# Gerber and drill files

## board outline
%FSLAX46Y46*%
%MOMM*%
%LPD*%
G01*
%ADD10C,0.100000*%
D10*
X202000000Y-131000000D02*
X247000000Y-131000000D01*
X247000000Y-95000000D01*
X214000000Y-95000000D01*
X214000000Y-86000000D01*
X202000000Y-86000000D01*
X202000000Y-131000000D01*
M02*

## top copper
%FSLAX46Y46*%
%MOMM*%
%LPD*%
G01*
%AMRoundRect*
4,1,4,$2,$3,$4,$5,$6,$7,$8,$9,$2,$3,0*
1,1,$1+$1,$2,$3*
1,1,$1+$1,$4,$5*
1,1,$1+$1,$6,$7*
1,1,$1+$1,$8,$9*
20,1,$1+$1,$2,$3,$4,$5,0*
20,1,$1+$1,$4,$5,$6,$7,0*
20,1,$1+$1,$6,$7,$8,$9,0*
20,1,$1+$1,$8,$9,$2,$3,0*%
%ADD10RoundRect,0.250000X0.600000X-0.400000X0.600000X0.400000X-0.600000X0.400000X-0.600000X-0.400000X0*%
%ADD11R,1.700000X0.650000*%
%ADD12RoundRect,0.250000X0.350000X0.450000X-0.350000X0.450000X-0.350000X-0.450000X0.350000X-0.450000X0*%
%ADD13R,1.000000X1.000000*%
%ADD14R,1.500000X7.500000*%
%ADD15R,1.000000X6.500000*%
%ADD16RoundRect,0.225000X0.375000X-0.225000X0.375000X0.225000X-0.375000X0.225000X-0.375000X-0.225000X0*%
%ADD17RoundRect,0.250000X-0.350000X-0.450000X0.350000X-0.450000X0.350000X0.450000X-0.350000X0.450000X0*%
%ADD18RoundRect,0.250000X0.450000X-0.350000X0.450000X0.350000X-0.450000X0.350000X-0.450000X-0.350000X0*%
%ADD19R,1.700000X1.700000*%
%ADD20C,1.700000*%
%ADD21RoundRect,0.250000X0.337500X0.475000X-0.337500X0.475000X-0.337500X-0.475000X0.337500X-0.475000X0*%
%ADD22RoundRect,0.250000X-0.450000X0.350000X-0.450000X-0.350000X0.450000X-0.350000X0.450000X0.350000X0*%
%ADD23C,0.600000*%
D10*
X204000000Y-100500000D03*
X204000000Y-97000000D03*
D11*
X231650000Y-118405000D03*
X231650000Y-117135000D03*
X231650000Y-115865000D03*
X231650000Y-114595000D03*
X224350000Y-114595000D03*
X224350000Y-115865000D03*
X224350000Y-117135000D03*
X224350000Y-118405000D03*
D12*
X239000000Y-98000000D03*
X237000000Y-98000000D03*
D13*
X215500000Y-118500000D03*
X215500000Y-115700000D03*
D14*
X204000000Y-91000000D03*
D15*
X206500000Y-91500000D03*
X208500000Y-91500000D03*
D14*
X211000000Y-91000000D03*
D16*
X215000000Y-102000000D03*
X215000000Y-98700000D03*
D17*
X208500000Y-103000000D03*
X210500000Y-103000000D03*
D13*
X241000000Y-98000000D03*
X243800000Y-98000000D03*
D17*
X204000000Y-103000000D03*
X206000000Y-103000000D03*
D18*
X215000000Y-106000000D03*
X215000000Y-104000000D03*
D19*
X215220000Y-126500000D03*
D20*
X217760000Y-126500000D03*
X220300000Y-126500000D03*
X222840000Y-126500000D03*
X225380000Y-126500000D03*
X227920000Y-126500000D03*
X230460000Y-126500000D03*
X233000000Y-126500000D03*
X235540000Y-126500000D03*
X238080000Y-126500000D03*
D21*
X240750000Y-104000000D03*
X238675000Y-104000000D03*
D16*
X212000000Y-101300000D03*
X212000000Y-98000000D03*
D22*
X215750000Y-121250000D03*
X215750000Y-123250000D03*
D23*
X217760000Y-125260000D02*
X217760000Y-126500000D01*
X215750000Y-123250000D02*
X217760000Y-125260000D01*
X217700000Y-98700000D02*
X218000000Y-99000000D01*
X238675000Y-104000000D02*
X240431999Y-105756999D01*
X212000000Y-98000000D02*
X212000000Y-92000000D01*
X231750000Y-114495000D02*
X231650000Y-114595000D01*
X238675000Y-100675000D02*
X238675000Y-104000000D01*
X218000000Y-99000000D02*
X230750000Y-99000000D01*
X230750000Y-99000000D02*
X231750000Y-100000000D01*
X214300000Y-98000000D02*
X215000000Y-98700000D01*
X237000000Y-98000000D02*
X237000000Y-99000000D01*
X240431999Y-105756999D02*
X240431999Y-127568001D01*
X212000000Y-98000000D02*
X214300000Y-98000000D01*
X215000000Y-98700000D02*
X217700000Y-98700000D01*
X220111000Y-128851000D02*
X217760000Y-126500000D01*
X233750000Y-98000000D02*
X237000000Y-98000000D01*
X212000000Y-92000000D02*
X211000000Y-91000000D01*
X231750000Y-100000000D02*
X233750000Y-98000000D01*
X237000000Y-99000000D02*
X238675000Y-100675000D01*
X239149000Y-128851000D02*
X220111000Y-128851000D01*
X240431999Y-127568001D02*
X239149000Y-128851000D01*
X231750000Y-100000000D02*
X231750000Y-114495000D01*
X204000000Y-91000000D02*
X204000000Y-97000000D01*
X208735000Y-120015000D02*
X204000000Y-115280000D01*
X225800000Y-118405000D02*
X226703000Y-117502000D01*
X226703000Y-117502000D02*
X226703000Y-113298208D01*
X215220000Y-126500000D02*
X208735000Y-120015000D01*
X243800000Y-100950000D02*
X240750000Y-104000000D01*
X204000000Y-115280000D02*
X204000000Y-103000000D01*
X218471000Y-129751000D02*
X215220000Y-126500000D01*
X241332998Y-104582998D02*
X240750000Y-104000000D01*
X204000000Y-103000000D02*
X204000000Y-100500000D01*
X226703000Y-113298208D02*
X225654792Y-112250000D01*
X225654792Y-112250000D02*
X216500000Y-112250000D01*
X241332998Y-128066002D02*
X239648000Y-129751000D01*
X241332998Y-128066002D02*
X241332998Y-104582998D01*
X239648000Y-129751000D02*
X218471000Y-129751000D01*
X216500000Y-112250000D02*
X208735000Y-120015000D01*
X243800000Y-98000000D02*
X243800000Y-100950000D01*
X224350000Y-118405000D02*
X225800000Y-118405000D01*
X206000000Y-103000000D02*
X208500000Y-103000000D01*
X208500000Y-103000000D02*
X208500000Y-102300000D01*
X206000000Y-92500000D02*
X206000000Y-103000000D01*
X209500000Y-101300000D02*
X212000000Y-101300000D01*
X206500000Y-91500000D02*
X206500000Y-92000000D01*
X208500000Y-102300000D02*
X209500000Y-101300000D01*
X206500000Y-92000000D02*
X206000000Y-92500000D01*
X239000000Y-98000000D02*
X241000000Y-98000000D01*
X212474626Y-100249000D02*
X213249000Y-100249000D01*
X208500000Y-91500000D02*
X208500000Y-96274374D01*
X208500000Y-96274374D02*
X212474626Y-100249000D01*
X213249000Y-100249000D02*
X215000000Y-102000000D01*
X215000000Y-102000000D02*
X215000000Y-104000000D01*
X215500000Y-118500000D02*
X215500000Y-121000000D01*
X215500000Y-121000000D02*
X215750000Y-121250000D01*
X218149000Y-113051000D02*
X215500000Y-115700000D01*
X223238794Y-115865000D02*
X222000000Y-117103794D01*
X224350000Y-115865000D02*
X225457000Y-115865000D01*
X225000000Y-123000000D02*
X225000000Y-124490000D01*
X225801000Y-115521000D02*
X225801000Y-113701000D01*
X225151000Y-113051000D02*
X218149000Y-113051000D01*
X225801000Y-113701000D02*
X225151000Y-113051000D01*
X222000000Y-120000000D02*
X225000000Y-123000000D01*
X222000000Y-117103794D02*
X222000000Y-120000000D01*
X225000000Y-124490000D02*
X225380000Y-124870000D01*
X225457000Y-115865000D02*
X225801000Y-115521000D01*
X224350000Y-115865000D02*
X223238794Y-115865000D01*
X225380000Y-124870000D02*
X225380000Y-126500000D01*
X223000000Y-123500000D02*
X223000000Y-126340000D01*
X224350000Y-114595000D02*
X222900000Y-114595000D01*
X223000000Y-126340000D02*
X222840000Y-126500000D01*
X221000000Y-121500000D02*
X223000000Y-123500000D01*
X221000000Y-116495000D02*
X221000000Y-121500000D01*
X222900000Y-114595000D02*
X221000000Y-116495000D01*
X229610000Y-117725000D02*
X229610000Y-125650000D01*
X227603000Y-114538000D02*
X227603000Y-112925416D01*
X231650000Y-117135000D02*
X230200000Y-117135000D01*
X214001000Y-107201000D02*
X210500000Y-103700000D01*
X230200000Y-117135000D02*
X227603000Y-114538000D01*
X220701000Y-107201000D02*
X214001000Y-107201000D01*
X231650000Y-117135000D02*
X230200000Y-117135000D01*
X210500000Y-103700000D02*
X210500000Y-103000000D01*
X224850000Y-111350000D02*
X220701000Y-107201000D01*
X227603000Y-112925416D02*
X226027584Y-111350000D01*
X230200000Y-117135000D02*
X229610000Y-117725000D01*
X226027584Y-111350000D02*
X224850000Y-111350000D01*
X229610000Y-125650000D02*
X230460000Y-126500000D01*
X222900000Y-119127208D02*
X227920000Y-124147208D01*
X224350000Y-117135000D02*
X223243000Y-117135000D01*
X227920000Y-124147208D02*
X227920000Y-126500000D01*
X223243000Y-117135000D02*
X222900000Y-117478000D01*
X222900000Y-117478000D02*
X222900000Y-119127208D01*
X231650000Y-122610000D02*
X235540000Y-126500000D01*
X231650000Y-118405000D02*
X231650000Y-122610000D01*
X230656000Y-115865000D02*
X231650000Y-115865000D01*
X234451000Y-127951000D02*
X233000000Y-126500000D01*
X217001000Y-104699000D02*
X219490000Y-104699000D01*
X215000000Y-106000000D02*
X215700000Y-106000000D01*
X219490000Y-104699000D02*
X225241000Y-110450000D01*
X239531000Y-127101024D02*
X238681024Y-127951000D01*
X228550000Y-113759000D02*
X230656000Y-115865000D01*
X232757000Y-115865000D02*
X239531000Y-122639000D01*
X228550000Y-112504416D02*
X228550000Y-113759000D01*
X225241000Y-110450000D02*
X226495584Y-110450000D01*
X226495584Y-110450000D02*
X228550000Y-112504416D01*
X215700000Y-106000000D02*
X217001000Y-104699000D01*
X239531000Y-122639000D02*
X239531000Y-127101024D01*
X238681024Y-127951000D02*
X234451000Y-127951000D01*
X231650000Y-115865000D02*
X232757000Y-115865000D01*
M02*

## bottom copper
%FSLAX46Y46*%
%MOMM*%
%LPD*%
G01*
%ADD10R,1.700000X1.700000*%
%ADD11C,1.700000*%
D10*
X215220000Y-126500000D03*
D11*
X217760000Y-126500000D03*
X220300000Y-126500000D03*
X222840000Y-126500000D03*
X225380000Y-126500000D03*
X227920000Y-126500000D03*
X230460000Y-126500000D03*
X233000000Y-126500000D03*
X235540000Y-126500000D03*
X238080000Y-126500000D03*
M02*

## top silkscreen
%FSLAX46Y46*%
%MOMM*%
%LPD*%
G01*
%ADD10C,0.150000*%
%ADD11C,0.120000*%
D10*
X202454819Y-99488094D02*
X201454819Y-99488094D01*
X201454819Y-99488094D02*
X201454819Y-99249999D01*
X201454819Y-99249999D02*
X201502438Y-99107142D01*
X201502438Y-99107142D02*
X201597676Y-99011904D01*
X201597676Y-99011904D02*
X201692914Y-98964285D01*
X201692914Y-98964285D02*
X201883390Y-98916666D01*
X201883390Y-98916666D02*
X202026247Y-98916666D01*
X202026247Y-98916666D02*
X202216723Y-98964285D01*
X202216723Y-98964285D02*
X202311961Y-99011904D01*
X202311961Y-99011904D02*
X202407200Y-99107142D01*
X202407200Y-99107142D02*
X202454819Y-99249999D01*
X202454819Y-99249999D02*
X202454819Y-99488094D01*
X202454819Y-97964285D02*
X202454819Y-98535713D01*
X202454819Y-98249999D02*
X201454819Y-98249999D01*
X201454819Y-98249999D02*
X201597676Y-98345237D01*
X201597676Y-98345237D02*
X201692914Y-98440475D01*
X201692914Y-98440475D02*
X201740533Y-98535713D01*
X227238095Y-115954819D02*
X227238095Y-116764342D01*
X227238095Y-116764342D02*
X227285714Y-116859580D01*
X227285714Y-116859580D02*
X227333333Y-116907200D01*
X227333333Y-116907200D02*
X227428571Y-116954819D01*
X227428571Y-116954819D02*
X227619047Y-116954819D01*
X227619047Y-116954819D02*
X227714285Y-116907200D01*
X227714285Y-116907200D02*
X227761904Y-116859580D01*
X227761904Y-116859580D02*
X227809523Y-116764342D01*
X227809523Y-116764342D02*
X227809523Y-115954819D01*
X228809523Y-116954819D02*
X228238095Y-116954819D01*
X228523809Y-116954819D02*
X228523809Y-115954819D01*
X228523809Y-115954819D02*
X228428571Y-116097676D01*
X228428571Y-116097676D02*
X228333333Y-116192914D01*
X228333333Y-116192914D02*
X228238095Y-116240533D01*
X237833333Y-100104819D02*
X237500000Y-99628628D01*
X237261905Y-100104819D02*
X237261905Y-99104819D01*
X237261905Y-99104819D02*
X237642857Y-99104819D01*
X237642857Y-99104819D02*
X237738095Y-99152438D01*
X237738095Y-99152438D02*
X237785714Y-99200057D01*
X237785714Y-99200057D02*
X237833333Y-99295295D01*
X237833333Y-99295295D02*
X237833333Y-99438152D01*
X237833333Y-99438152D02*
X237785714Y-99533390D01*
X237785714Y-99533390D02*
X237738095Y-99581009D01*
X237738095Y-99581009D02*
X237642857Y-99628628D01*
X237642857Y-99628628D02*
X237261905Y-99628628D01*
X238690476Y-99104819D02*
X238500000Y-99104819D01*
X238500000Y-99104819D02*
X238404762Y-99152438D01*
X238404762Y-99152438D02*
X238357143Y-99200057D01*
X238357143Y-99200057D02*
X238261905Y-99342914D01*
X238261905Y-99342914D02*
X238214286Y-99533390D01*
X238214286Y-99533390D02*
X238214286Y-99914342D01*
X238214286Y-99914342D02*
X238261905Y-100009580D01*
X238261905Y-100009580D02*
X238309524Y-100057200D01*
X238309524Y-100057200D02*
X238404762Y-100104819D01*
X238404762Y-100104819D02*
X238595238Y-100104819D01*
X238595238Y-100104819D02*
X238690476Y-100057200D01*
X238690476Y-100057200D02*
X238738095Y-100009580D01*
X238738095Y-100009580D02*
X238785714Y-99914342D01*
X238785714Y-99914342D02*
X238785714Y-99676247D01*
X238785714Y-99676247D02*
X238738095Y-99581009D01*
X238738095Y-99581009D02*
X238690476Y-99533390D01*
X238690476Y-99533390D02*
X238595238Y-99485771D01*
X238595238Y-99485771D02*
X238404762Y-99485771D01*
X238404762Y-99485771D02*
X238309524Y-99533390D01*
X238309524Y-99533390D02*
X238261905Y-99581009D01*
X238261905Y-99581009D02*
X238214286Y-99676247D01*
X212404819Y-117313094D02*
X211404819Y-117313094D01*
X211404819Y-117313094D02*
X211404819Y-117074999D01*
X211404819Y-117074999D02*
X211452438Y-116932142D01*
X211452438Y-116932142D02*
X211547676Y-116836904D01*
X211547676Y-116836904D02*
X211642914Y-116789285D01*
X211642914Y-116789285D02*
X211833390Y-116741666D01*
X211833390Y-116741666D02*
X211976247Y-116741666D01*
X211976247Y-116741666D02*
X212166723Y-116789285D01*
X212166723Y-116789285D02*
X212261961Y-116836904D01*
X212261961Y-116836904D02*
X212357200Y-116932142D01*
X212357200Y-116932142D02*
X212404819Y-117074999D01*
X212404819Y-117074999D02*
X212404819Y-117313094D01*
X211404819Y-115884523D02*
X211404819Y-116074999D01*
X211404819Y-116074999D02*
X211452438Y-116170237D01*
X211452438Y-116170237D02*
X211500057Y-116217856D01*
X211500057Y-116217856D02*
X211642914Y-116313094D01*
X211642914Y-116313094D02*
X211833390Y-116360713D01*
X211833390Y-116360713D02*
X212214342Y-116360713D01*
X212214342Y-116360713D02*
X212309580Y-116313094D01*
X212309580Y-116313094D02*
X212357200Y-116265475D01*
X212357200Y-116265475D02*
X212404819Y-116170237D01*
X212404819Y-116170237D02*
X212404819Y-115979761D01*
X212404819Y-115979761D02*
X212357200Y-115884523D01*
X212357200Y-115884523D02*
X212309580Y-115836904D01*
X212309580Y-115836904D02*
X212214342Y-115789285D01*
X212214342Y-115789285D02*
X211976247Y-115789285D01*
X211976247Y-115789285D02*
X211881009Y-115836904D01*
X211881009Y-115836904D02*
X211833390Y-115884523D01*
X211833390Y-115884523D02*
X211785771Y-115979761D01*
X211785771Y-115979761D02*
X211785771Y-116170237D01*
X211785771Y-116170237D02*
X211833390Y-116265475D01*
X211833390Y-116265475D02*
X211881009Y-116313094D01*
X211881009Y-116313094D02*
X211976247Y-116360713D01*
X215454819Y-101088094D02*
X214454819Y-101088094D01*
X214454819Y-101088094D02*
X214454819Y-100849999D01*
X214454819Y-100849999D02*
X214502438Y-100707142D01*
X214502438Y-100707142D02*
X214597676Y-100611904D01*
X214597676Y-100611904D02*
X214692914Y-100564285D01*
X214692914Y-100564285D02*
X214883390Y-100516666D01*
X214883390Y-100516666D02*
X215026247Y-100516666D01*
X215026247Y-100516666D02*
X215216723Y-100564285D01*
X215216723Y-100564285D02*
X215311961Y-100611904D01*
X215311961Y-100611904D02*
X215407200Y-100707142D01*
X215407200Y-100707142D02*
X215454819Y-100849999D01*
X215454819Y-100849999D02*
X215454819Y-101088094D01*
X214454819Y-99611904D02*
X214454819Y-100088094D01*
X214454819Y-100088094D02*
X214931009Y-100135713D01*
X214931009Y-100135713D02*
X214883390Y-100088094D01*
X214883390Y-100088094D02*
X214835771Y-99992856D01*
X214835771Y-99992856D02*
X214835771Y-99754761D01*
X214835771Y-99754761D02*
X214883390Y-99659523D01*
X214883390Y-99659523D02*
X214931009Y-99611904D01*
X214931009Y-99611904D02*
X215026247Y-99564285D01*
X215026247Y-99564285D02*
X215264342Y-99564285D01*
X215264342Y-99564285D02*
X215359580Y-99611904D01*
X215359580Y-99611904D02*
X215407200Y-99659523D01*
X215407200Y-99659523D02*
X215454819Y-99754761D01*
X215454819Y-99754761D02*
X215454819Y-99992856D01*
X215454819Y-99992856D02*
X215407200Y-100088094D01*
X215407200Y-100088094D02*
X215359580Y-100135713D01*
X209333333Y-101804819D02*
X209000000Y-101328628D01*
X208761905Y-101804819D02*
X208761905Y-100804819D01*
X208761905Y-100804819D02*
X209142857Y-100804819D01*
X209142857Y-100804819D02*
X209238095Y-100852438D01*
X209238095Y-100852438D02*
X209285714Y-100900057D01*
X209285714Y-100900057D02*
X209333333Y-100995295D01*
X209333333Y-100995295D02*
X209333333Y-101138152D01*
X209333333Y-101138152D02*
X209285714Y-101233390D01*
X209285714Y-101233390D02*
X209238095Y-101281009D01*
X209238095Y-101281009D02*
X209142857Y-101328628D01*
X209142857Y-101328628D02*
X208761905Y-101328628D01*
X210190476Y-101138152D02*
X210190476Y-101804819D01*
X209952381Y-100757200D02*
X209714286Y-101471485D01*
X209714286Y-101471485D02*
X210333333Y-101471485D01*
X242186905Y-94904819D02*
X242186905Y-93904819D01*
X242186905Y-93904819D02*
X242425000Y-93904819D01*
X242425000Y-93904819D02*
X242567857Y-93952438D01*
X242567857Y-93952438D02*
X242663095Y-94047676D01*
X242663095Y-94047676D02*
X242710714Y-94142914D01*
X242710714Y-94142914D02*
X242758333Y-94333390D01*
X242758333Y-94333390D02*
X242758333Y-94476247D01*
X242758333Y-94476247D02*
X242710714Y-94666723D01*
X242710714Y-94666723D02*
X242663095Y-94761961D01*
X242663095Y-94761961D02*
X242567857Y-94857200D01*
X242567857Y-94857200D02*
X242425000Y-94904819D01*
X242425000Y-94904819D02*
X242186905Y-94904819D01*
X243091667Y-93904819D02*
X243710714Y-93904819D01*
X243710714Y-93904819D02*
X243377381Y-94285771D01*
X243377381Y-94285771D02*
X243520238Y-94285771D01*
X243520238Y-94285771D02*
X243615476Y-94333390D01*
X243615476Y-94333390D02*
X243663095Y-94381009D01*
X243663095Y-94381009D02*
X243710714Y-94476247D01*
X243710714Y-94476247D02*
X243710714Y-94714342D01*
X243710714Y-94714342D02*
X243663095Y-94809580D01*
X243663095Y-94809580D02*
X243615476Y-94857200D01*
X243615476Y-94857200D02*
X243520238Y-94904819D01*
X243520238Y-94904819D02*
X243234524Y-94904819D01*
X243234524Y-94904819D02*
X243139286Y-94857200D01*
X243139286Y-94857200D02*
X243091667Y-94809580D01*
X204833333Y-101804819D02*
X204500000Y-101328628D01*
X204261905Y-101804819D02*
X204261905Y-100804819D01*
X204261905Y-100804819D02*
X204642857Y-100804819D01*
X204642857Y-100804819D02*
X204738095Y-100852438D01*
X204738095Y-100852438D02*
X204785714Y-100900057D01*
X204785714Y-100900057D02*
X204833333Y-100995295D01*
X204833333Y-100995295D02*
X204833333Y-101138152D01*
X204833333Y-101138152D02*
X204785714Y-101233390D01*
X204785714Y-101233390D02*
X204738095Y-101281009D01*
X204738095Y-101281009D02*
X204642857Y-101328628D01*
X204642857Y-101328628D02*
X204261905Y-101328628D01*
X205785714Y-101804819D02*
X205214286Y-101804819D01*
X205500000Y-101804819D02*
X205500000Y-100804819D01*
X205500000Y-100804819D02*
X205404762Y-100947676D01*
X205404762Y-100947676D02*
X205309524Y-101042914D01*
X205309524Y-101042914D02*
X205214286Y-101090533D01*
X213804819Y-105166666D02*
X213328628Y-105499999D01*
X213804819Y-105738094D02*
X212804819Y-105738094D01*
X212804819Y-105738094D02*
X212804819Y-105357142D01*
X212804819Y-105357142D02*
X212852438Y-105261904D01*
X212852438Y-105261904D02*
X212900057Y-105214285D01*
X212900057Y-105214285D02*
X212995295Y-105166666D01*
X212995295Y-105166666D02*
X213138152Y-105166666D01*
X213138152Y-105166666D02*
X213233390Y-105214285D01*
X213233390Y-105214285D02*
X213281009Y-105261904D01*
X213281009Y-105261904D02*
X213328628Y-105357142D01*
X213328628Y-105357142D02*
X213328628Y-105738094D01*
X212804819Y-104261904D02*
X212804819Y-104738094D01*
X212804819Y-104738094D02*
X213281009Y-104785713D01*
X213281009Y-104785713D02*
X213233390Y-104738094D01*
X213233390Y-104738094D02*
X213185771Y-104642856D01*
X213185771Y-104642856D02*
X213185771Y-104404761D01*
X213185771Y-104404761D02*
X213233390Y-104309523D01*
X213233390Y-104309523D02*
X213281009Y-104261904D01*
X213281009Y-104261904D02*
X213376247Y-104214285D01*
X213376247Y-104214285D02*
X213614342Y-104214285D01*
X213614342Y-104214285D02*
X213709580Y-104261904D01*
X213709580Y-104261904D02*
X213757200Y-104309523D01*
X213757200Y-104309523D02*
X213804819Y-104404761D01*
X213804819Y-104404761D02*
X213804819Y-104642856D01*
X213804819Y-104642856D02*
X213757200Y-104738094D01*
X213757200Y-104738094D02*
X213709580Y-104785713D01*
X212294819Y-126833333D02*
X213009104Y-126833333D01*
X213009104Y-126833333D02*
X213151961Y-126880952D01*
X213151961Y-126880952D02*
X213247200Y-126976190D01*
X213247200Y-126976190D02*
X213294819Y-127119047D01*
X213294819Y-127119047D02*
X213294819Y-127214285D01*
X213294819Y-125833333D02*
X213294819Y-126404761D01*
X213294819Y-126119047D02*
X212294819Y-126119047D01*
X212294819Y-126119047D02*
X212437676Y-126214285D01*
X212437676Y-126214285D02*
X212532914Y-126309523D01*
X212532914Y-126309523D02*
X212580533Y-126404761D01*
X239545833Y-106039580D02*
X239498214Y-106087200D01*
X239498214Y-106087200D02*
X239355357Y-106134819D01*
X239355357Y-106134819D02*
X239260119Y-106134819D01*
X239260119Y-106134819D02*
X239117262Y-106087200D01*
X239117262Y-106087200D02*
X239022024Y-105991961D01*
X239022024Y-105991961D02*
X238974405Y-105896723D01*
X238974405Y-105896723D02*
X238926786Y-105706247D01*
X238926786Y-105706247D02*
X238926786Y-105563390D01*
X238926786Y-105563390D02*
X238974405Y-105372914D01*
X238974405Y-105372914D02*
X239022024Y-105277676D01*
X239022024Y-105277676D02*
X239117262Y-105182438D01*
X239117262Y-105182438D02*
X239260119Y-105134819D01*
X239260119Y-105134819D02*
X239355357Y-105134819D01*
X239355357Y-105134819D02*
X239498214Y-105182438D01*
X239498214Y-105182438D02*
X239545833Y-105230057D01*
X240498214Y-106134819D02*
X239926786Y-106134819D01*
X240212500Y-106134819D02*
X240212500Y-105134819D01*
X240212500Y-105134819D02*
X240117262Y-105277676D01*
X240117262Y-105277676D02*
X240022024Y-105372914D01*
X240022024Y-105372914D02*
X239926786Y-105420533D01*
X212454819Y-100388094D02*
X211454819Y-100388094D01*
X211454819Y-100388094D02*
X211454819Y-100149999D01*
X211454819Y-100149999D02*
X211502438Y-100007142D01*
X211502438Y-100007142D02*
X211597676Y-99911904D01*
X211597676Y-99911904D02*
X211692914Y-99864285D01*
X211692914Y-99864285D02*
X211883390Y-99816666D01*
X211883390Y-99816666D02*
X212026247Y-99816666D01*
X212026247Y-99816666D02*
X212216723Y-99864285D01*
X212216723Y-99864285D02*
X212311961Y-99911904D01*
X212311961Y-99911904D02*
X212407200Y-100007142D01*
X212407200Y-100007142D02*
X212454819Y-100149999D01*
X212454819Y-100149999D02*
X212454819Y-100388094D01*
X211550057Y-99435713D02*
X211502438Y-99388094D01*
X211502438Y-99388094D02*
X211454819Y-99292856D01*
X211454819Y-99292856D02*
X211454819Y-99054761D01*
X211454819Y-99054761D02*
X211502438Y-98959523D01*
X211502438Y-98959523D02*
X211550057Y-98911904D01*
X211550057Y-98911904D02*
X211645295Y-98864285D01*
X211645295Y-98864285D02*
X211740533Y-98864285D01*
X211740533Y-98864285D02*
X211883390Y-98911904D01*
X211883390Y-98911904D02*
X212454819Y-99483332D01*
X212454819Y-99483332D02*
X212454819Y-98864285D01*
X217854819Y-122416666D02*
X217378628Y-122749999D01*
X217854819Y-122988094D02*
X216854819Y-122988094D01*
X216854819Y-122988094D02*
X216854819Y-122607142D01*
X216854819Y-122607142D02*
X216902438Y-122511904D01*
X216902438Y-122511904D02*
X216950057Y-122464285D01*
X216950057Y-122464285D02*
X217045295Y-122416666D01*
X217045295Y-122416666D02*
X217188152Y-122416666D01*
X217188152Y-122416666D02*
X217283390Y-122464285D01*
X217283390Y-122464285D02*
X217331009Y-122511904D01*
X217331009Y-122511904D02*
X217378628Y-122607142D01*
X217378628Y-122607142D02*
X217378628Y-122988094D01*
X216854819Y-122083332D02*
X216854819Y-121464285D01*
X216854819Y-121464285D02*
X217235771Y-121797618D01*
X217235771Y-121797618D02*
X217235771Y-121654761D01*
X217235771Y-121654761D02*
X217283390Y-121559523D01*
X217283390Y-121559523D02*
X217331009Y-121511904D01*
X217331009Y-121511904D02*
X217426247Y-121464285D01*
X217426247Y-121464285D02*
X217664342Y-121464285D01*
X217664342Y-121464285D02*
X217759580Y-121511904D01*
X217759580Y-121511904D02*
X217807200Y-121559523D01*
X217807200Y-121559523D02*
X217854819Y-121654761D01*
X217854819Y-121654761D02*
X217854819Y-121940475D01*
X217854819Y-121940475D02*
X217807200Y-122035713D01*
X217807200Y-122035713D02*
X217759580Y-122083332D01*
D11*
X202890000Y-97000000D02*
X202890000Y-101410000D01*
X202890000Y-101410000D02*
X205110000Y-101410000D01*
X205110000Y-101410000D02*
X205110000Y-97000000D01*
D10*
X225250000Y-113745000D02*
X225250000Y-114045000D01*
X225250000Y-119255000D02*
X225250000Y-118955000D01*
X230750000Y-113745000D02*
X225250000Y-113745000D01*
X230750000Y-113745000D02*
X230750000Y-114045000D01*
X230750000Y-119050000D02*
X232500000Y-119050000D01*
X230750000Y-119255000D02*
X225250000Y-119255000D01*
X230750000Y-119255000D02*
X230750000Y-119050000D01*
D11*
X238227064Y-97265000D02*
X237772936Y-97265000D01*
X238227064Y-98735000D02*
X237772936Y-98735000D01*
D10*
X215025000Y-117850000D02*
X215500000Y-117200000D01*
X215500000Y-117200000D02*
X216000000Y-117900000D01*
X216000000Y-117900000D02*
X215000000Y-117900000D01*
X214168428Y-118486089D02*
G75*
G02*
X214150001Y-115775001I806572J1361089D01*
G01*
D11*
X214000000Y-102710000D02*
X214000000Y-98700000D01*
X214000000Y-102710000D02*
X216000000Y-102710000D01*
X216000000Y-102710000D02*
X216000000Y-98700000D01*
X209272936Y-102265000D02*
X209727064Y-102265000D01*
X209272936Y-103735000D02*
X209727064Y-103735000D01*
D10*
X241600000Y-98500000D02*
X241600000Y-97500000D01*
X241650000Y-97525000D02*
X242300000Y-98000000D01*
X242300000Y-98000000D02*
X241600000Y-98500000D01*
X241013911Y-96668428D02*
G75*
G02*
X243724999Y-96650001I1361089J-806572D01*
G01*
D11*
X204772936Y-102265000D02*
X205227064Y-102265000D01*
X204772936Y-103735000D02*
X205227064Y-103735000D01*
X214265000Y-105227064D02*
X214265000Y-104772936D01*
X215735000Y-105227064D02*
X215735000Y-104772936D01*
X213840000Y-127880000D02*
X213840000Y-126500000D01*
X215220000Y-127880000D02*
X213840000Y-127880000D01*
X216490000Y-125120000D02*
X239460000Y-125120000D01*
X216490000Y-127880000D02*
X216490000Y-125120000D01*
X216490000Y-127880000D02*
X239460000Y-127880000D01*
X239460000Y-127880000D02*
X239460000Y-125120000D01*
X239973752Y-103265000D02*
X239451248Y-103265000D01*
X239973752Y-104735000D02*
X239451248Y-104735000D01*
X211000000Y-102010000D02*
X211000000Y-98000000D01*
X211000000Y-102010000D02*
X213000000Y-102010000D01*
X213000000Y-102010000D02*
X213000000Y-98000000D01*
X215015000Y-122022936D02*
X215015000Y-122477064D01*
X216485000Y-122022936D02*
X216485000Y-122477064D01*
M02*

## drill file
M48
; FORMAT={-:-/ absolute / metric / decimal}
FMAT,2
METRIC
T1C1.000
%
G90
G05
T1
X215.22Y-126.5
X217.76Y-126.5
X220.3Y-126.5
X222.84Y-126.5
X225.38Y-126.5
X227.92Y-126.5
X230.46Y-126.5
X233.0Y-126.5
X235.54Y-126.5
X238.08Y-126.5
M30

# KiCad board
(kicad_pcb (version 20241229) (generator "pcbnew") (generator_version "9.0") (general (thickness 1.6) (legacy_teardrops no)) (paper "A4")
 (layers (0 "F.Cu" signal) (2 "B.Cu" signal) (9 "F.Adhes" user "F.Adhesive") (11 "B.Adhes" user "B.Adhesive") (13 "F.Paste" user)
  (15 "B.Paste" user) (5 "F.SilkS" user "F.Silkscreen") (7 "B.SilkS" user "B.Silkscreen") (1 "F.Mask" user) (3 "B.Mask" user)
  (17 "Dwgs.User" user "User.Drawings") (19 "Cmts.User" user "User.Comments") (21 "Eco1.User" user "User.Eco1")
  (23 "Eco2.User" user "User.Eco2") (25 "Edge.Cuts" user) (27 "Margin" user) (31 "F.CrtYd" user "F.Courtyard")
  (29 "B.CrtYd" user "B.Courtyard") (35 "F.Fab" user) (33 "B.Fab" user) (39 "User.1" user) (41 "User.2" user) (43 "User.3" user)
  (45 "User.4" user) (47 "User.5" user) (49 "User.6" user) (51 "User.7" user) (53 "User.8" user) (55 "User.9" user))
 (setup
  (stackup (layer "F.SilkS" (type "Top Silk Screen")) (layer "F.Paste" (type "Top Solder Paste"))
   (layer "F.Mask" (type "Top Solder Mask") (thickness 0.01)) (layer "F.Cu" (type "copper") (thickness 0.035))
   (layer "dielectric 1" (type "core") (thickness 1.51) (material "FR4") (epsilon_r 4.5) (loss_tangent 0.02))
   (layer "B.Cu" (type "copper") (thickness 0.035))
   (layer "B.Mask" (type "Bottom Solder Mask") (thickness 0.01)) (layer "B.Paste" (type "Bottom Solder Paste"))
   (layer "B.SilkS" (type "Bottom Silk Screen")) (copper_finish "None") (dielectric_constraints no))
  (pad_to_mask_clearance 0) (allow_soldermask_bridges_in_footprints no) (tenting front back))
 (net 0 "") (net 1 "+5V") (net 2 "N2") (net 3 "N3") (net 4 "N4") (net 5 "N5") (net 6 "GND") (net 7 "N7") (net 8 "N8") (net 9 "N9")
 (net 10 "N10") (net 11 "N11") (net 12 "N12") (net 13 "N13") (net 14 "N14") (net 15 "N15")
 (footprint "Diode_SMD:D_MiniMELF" (layer "F.Cu") (at 204 98.75 90)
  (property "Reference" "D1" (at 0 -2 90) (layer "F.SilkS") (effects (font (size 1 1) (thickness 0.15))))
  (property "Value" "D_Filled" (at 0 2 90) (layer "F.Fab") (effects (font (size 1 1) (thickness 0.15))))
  (fp_line (start 1.75 -1.11) (end -2.66 -1.11) (stroke (width 0.12) (type solid)) (layer "F.SilkS"))
  (fp_line (start -2.66 -1.11) (end -2.66 1.11) (stroke (width 0.12) (type solid)) (layer "F.SilkS"))
  (fp_line (start -2.66 1.11) (end 1.75 1.11) (stroke (width 0.12) (type solid)) (layer "F.SilkS"))
  (pad "1" smd roundrect (at -1.75 0 90) (size 1.3 1.7) (layers "F.Cu" "F.Mask" "F.Paste") (roundrect_rratio 0.1923076923) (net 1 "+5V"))
  (pad "2" smd roundrect (at 1.75 0 90) (size 1.3 1.7) (layers "F.Cu" "F.Mask" "F.Paste") (roundrect_rratio 0.1923076923) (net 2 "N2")))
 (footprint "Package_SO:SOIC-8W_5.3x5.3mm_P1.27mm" (layer "F.Cu") (at 228 116.5 180)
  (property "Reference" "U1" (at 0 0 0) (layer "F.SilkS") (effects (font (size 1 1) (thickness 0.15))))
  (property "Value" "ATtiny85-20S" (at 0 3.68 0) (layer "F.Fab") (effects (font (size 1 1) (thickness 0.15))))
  (fp_line (start 2.75 2.755) (end 2.75 2.455) (stroke (width 0.15) (type solid)) (layer "F.SilkS"))
  (fp_line (start 2.75 -2.755) (end 2.75 -2.455) (stroke (width 0.15) (type solid)) (layer "F.SilkS"))
  (fp_line (start -2.75 2.755) (end 2.75 2.755) (stroke (width 0.15) (type solid)) (layer "F.SilkS"))
  (fp_line (start -2.75 2.755) (end -2.75 2.455) (stroke (width 0.15) (type solid)) (layer "F.SilkS"))
  (fp_line (start -2.75 -2.55) (end -4.5 -2.55) (stroke (width 0.15) (type solid)) (layer "F.SilkS"))
  (fp_line (start -2.75 -2.755) (end 2.75 -2.755) (stroke (width 0.15) (type solid)) (layer "F.SilkS"))
  (fp_line (start -2.75 -2.755) (end -2.75 -2.55) (stroke (width 0.15) (type solid)) (layer "F.SilkS"))
  (pad "1" smd rect (at -3.65 -1.905 180) (size 1.7 0.65) (layers "F.Cu" "F.Mask" "F.Paste") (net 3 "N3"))
  (pad "2" smd rect (at -3.65 -0.635 180) (size 1.7 0.65) (layers "F.Cu" "F.Mask" "F.Paste") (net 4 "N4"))
  (pad "3" smd rect (at -3.65 0.635 180) (size 1.7 0.65) (layers "F.Cu" "F.Mask" "F.Paste") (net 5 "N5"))
  (pad "4" smd rect (at -3.65 1.905 180) (size 1.7 0.65) (layers "F.Cu" "F.Mask" "F.Paste") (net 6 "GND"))
  (pad "5" smd rect (at 3.65 1.905 180) (size 1.7 0.65) (layers "F.Cu" "F.Mask" "F.Paste") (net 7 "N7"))
  (pad "6" smd rect (at 3.65 0.635 180) (size 1.7 0.65) (layers "F.Cu" "F.Mask" "F.Paste") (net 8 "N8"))
  (pad "7" smd rect (at 3.65 -0.635 180) (size 1.7 0.65) (layers "F.Cu" "F.Mask" "F.Paste") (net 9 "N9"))
  (pad "8" smd rect (at 3.65 -1.905 180) (size 1.7 0.65) (layers "F.Cu" "F.Mask" "F.Paste") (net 1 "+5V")))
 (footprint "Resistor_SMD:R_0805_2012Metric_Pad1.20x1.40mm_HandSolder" (layer "F.Cu") (at 238 98 180)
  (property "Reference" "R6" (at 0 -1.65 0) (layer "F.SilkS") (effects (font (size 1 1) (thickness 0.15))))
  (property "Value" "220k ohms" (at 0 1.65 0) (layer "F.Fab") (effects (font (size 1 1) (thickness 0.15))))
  (fp_line (start -0.227064 0.735) (end 0.227064 0.735) (stroke (width 0.12) (type solid)) (layer "F.SilkS"))
  (fp_line (start -0.227064 -0.735) (end 0.227064 -0.735) (stroke (width 0.12) (type solid)) (layer "F.SilkS"))
  (pad "1" smd roundrect (at -1 0 180) (size 1.2 1.4) (layers "F.Cu" "F.Mask" "F.Paste") (roundrect_rratio 0.208333) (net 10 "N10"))
  (pad "2" smd roundrect (at 1 0 180) (size 1.2 1.4) (layers "F.Cu" "F.Mask" "F.Paste") (roundrect_rratio 0.208333) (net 6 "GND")))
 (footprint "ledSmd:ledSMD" (layer "F.Cu") (at 215.5 116.7 90)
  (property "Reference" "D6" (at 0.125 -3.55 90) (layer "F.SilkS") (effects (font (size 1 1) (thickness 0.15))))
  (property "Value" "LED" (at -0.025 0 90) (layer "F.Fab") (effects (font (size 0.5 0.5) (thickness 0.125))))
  (fp_line (start -1.15 -0.475) (end -0.5 0) (stroke (width 0.15) (type solid)) (layer "F.SilkS"))
  (fp_line (start -0.5 0) (end -1.2 0.5) (stroke (width 0.15) (type solid)) (layer "F.SilkS"))
  (fp_line (start -1.2 0.5) (end -1.2 -0.5) (stroke (width 0.15) (type solid)) (layer "F.SilkS"))
  (fp_arc (start -1.786089 -1.331572) (mid -0.435753 -2.107089) (end 0.924999 -1.349999) (stroke (width 0.15) (type solid))
   (layer "F.SilkS"))
  (pad "1" smd rect (at -1.8 0 90) (size 1 1) (layers "F.Cu" "F.Mask" "F.Paste") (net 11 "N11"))
  (pad "2" smd rect (at 1 0 90) (size 1 1) (layers "F.Cu" "F.Mask" "F.Paste") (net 8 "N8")))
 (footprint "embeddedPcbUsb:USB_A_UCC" (layer "F.Cu") (at 207.5 91.2 -90)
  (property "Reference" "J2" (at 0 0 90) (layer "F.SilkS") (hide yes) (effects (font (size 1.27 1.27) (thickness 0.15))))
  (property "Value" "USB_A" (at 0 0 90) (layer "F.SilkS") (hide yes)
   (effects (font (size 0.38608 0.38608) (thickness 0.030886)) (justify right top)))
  (pad "1" smd rect (at -0.2 3.5 270) (size 7.5 1.5) (layers "F.Cu" "F.Mask" "F.Paste") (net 2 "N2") (solder_mask_margin 0.1016))
  (pad "2" smd rect (at 0.3 1 270) (size 6.5 1) (layers "F.Cu" "F.Mask" "F.Paste") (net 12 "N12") (solder_mask_margin 0.1016))
  (pad "3" smd rect (at 0.3 -1 270) (size 6.5 1) (layers "F.Cu" "F.Mask" "F.Paste") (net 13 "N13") (solder_mask_margin 0.1016))
  (pad "4" smd rect (at -0.2 -3.5 270) (size 7.5 1.5) (layers "F.Cu" "F.Mask" "F.Paste") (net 6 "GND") (solder_mask_margin 0.1016)))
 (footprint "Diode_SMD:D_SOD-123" (layer "F.Cu") (at 215 100.35 90)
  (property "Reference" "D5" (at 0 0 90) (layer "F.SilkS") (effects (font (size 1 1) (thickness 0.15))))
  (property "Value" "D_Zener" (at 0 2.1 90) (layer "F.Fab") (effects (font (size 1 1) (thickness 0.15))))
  (fp_line (start -2.36 -1) (end 1.65 -1) (stroke (width 0.12) (type solid)) (layer "F.SilkS"))
  (fp_line (start -2.36 -1) (end -2.36 1) (stroke (width 0.12) (type solid)) (layer "F.SilkS"))
  (fp_line (start -2.36 1) (end 1.65 1) (stroke (width 0.12) (type solid)) (layer "F.SilkS"))
  (pad "1" smd roundrect (at -1.65 0 90) (size 0.9 1.2) (layers "F.Cu" "F.Mask" "F.Paste") (roundrect_rratio 0.25) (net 13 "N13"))
  (pad "2" smd roundrect (at 1.65 0 90) (size 0.9 1.2) (layers "F.Cu" "F.Mask" "F.Paste") (roundrect_rratio 0.25) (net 6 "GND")))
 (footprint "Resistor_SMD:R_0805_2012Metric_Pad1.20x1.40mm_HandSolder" (layer "F.Cu") (at 209.5 103)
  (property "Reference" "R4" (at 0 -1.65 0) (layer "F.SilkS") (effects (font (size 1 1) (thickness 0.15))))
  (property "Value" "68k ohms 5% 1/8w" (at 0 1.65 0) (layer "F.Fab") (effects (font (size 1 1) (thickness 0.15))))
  (fp_line (start -0.227064 -0.735) (end 0.227064 -0.735) (stroke (width 0.12) (type solid)) (layer "F.SilkS"))
  (fp_line (start -0.227064 0.735) (end 0.227064 0.735) (stroke (width 0.12) (type solid)) (layer "F.SilkS"))
  (pad "1" smd roundrect (at -1 0) (size 1.2 1.4) (layers "F.Cu" "F.Mask" "F.Paste") (roundrect_rratio 0.208333) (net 12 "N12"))
  (pad "2" smd roundrect (at 1 0) (size 1.2 1.4) (layers "F.Cu" "F.Mask" "F.Paste") (roundrect_rratio 0.208333) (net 4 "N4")))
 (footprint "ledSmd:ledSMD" (layer "F.Cu") (at 242.8 98)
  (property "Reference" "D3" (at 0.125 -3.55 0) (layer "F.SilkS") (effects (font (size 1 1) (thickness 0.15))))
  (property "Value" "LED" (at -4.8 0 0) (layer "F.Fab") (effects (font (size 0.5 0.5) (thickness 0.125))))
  (fp_line (start -1.2 0.5) (end -1.2 -0.5) (stroke (width 0.15) (type solid)) (layer "F.SilkS"))
  (fp_line (start -1.15 -0.475) (end -0.5 0) (stroke (width 0.15) (type solid)) (layer "F.SilkS"))
  (fp_line (start -0.5 0) (end -1.2 0.5) (stroke (width 0.15) (type solid)) (layer "F.SilkS"))
  (fp_arc (start -1.786089 -1.331572) (mid -0.435753 -2.107089) (end 0.924999 -1.349999) (stroke (width 0.15) (type solid))
   (layer "F.SilkS"))
  (pad "1" smd rect (at -1.8 0) (size 1 1) (layers "F.Cu" "F.Mask" "F.Paste") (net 10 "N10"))
  (pad "2" smd rect (at 1 0) (size 1 1) (layers "F.Cu" "F.Mask" "F.Paste") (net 1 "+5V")))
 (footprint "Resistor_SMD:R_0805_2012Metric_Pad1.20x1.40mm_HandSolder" (layer "F.Cu") (at 205 103)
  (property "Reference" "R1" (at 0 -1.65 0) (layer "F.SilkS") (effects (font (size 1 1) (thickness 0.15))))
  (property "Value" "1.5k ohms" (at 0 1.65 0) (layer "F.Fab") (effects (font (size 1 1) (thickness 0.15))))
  (fp_line (start -0.227064 -0.735) (end 0.227064 -0.735) (stroke (width 0.12) (type solid)) (layer "F.SilkS"))
  (fp_line (start -0.227064 0.735) (end 0.227064 0.735) (stroke (width 0.12) (type solid)) (layer "F.SilkS"))
  (pad "1" smd roundrect (at -1 0) (size 1.2 1.4) (layers "F.Cu" "F.Mask" "F.Paste") (roundrect_rratio 0.208333) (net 1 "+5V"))
  (pad "2" smd roundrect (at 1 0) (size 1.2 1.4) (layers "F.Cu" "F.Mask" "F.Paste") (roundrect_rratio 0.208333) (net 12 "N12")))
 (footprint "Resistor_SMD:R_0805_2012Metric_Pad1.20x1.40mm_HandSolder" (layer "F.Cu") (at 215 105 90)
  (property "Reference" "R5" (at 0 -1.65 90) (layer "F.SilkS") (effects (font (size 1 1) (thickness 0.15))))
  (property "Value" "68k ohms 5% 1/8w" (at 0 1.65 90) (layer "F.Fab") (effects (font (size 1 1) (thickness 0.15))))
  (fp_line (start -0.227064 -0.735) (end 0.227064 -0.735) (stroke (width 0.12) (type solid)) (layer "F.SilkS"))
  (fp_line (start -0.227064 0.735) (end 0.227064 0.735) (stroke (width 0.12) (type solid)) (layer "F.SilkS"))
  (pad "1" smd roundrect (at -1 0 90) (size 1.2 1.4) (layers "F.Cu" "F.Mask" "F.Paste") (roundrect_rratio 0.208333) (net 5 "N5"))
  (pad "2" smd roundrect (at 1 0 90) (size 1.2 1.4) (layers "F.Cu" "F.Mask" "F.Paste") (roundrect_rratio 0.208333) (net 13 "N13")))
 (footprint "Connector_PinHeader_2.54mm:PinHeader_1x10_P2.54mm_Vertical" (layer "F.Cu") (at 215.22 126.5 90)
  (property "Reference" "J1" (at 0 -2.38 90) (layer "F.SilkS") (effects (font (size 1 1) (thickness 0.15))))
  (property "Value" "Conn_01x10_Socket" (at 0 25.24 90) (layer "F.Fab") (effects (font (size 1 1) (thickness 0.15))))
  (fp_line (start -1.38 -1.38) (end 0 -1.38) (stroke (width 0.12) (type solid)) (layer "F.SilkS"))
  (fp_line (start -1.38 0) (end -1.38 -1.38) (stroke (width 0.12) (type solid)) (layer "F.SilkS"))
  (fp_line (start 1.38 1.27) (end 1.38 24.24) (stroke (width 0.12) (type solid)) (layer "F.SilkS"))
  (fp_line (start -1.38 1.27) (end 1.38 1.27) (stroke (width 0.12) (type solid)) (layer "F.SilkS"))
  (fp_line (start -1.38 1.27) (end -1.38 24.24) (stroke (width 0.12) (type solid)) (layer "F.SilkS"))
  (fp_line (start -1.38 24.24) (end 1.38 24.24) (stroke (width 0.12) (type solid)) (layer "F.SilkS"))
  (pad "1" thru_hole rect (at 0 0 90) (size 1.7 1.7) (drill 1) (layers "*.Cu" "*.Mask") (remove_unused_layers no) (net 1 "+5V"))
  (pad "2" thru_hole circle (at 0 2.54 90) (size 1.7 1.7) (drill 1) (layers "*.Cu" "*.Mask") (remove_unused_layers no) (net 6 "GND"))
  (pad "3" thru_hole circle (at 0 5.08 90) (size 1.7 1.7) (drill 1) (layers "*.Cu" "*.Mask") (remove_unused_layers no) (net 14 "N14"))
  (pad "4" thru_hole circle (at 0 7.62 90) (size 1.7 1.7) (drill 1) (layers "*.Cu" "*.Mask") (remove_unused_layers no) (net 7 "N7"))
  (pad "5" thru_hole circle (at 0 10.16 90) (size 1.7 1.7) (drill 1) (layers "*.Cu" "*.Mask") (remove_unused_layers no) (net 8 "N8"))
  (pad "6" thru_hole circle (at 0 12.7 90) (size 1.7 1.7) (drill 1) (layers "*.Cu" "*.Mask") (remove_unused_layers no) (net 9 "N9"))
  (pad "7" thru_hole circle (at 0 15.24 90) (size 1.7 1.7) (drill 1) (layers "*.Cu" "*.Mask") (remove_unused_layers no) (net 4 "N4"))
  (pad "8" thru_hole circle (at 0 17.78 90) (size 1.7 1.7) (drill 1) (layers "*.Cu" "*.Mask") (remove_unused_layers no) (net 5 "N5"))
  (pad "9" thru_hole circle (at 0 20.32 90) (size 1.7 1.7) (drill 1) (layers "*.Cu" "*.Mask") (remove_unused_layers no) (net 3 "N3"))
  (pad "10" thru_hole circle (at 0 22.86 90) (size 1.7 1.7) (drill 1) (layers "*.Cu" "*.Mask") (remove_unused_layers no) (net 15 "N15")))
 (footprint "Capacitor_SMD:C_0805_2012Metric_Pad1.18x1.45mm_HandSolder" (layer "F.Cu") (at 239.7125 104 180)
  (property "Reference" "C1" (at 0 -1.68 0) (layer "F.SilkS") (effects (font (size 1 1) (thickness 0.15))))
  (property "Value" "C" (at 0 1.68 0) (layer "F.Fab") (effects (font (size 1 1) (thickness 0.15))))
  (fp_line (start -0.261252 0.735) (end 0.261252 0.735) (stroke (width 0.12) (type solid)) (layer "F.SilkS"))
  (fp_line (start -0.261252 -0.735) (end 0.261252 -0.735) (stroke (width 0.12) (type solid)) (layer "F.SilkS"))
  (pad "1" smd roundrect (at -1.0375 0 180) (size 1.175 1.45) (layers "F.Cu" "F.Mask" "F.Paste") (roundrect_rratio 0.212766) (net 1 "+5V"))
  (pad "2" smd roundrect (at 1.0375 0 180) (size 1.175 1.45) (layers "F.Cu" "F.Mask" "F.Paste") (roundrect_rratio 0.212766) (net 6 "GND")))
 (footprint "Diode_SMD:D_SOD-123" (layer "F.Cu") (at 212 99.65 90)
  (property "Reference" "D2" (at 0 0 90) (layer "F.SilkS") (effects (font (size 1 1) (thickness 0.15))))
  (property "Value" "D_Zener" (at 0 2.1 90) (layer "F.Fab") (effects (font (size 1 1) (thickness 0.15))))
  (fp_line (start -2.36 -1) (end 1.65 -1) (stroke (width 0.12) (type solid)) (layer "F.SilkS"))
  (fp_line (start -2.36 -1) (end -2.36 1) (stroke (width 0.12) (type solid)) (layer "F.SilkS"))
  (fp_line (start -2.36 1) (end 1.65 1) (stroke (width 0.12) (type solid)) (layer "F.SilkS"))
  (pad "1" smd roundrect (at -1.65 0 90) (size 0.9 1.2) (layers "F.Cu" "F.Mask" "F.Paste") (roundrect_rratio 0.25) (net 12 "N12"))
  (pad "2" smd roundrect (at 1.65 0 90) (size 0.9 1.2) (layers "F.Cu" "F.Mask" "F.Paste") (roundrect_rratio 0.25) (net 6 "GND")))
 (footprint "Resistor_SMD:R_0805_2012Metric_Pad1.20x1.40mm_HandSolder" (layer "F.Cu") (at 215.75 122.25 -90)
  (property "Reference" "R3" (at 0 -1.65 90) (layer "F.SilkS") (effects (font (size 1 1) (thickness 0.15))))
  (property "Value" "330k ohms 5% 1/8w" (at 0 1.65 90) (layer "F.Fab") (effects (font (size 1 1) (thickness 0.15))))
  (fp_line (start -0.227064 0.735) (end 0.227064 0.735) (stroke (width 0.12) (type solid)) (layer "F.SilkS"))
  (fp_line (start -0.227064 -0.735) (end 0.227064 -0.735) (stroke (width 0.12) (type solid)) (layer "F.SilkS"))
  (pad "1" smd roundrect (at -1 0 270) (size 1.2 1.4) (layers "F.Cu" "F.Mask" "F.Paste") (roundrect_rratio 0.208333) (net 11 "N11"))
  (pad "2" smd roundrect (at 1 0 270) (size 1.2 1.4) (layers "F.Cu" "F.Mask" "F.Paste") (roundrect_rratio 0.208333) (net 6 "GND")))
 (gr_poly
  (pts (xy 202 131) (xy 247 131) (xy 247 95) (xy 214 95) (xy 214 86) (xy 202 86)) (stroke (width 0.1) (type solid)) (fill no)
  (layer "Edge.Cuts"))
 (segment (start 217.76 125.26) (end 217.76 126.5) (width 0.6) (layer "F.Cu") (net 6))
 (segment (start 215.75 123.25) (end 217.76 125.26) (width 0.6) (layer "F.Cu") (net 6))
 (segment (start 217.7 98.7) (end 218 99) (width 0.6) (layer "F.Cu") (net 6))
 (segment (start 238.675 104) (end 240.431999 105.756999) (width 0.6) (layer "F.Cu") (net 6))
 (segment (start 212 98) (end 212 92) (width 0.6) (layer "F.Cu") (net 6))
 (segment (start 231.75 114.495) (end 231.65 114.595) (width 0.6) (layer "F.Cu") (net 6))
 (segment (start 238.675 100.675) (end 238.675 104) (width 0.6) (layer "F.Cu") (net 6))
 (segment (start 218 99) (end 230.75 99) (width 0.6) (layer "F.Cu") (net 6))
 (segment (start 230.75 99) (end 231.75 100) (width 0.6) (layer "F.Cu") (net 6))
 (segment (start 214.3 98) (end 215 98.7) (width 0.6) (layer "F.Cu") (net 6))
 (segment (start 237 98) (end 237 99) (width 0.6) (layer "F.Cu") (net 6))
 (segment (start 240.431999 105.756999) (end 240.431999 127.568001) (width 0.6) (layer "F.Cu") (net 6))
 (segment (start 212 98) (end 214.3 98) (width 0.6) (layer "F.Cu") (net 6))
 (segment (start 215 98.7) (end 217.7 98.7) (width 0.6) (layer "F.Cu") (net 6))
 (segment (start 220.111 128.851) (end 217.76 126.5) (width 0.6) (layer "F.Cu") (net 6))
 (segment (start 233.75 98) (end 237 98) (width 0.6) (layer "F.Cu") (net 6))
 (segment (start 212 92) (end 211 91) (width 0.6) (layer "F.Cu") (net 6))
 (segment (start 231.75 100) (end 233.75 98) (width 0.6) (layer "F.Cu") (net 6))
 (segment (start 237 99) (end 238.675 100.675) (width 0.6) (layer "F.Cu") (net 6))
 (segment (start 239.149 128.851) (end 220.111 128.851) (width 0.6) (layer "F.Cu") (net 6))
 (segment (start 240.431999 127.568001) (end 239.149 128.851) (width 0.6) (layer "F.Cu") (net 6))
 (segment (start 231.75 100) (end 231.75 114.495) (width 0.6) (layer "F.Cu") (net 6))
 (segment (start 204 91) (end 204 97) (width 0.6) (layer "F.Cu") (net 2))
 (segment (start 208.735 120.015) (end 204 115.28) (width 0.6) (layer "F.Cu") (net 1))
 (segment (start 225.8 118.405) (end 226.703 117.502) (width 0.6) (layer "F.Cu") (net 1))
 (segment (start 226.703 117.502) (end 226.703 113.298208) (width 0.6) (layer "F.Cu") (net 1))
 (segment (start 215.22 126.5) (end 208.735 120.015) (width 0.6) (layer "F.Cu") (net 1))
 (segment (start 243.8 100.95) (end 240.75 104) (width 0.6) (layer "F.Cu") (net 1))
 (segment (start 204 115.28) (end 204 103) (width 0.6) (layer "F.Cu") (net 1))
 (segment (start 218.471 129.751) (end 215.22 126.5) (width 0.6) (layer "F.Cu") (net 1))
 (segment (start 241.332998 104.582998) (end 240.75 104) (width 0.6) (layer "F.Cu") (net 1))
 (segment (start 204 103) (end 204 100.5) (width 0.6) (layer "F.Cu") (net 1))
 (segment (start 226.703 113.298208) (end 225.654792 112.25) (width 0.6) (layer "F.Cu") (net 1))
 (segment (start 225.654792 112.25) (end 216.5 112.25) (width 0.6) (layer "F.Cu") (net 1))
 (segment (start 241.332998 128.066002) (end 239.648 129.751) (width 0.6) (layer "F.Cu") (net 1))
 (segment (start 241.332998 128.066002) (end 241.332998 104.582998) (width 0.6) (layer "F.Cu") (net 1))
 (segment (start 239.648 129.751) (end 218.471 129.751) (width 0.6) (layer "F.Cu") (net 1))
 (segment (start 216.5 112.25) (end 208.735 120.015) (width 0.6) (layer "F.Cu") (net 1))
 (segment (start 243.8 98) (end 243.8 100.95) (width 0.6) (layer "F.Cu") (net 1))
 (segment (start 224.35 118.405) (end 225.8 118.405) (width 0.6) (layer "F.Cu") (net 1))
 (segment (start 206 103) (end 208.5 103) (width 0.6) (layer "F.Cu") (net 12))
 (segment (start 208.5 103) (end 208.5 102.3) (width 0.6) (layer "F.Cu") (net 12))
 (segment (start 206 92.5) (end 206 103) (width 0.6) (layer "F.Cu") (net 12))
 (segment (start 209.5 101.3) (end 212 101.3) (width 0.6) (layer "F.Cu") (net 12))
 (segment (start 206.5 91.5) (end 206.5 92) (width 0.6) (layer "F.Cu") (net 12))
 (segment (start 208.5 102.3) (end 209.5 101.3) (width 0.6) (layer "F.Cu") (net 12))
 (segment (start 206.5 92) (end 206 92.5) (width 0.6) (layer "F.Cu") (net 12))
 (segment (start 239 98) (end 241 98) (width 0.6) (layer "F.Cu") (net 10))
 (segment (start 212.474626 100.249) (end 213.249 100.249) (width 0.6) (layer "F.Cu") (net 13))
 (segment (start 208.5 91.5) (end 208.5 96.274374) (width 0.6) (layer "F.Cu") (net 13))
 (segment (start 208.5 96.274374) (end 212.474626 100.249) (width 0.6) (layer "F.Cu") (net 13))
 (segment (start 213.249 100.249) (end 215 102) (width 0.6) (layer "F.Cu") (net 13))
 (segment (start 215 102) (end 215 104) (width 0.6) (layer "F.Cu") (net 13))
 (segment (start 215.5 118.5) (end 215.5 121) (width 0.6) (layer "F.Cu") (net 11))
 (segment (start 215.5 121) (end 215.75 121.25) (width 0.6) (layer "F.Cu") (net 11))
 (segment (start 218.149 113.051) (end 215.5 115.7) (width 0.6) (layer "F.Cu") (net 8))
 (segment (start 223.238794 115.865) (end 222 117.103794) (width 0.6) (layer "F.Cu") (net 8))
 (segment (start 224.35 115.865) (end 225.457 115.865) (width 0.6) (layer "F.Cu") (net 8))
 (segment (start 225 123) (end 225 124.49) (width 0.6) (layer "F.Cu") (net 8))
 (segment (start 225.801 115.521) (end 225.801 113.701) (width 0.6) (layer "F.Cu") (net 8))
 (segment (start 225.151 113.051) (end 218.149 113.051) (width 0.6) (layer "F.Cu") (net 8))
 (segment (start 225.801 113.701) (end 225.151 113.051) (width 0.6) (layer "F.Cu") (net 8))
 (segment (start 222 120) (end 225 123) (width 0.6) (layer "F.Cu") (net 8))
 (segment (start 222 117.103794) (end 222 120) (width 0.6) (layer "F.Cu") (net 8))
 (segment (start 225 124.49) (end 225.38 124.87) (width 0.6) (layer "F.Cu") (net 8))
 (segment (start 225.457 115.865) (end 225.801 115.521) (width 0.6) (layer "F.Cu") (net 8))
 (segment (start 224.35 115.865) (end 223.238794 115.865) (width 0.6) (layer "F.Cu") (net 8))
 (segment (start 225.38 124.87) (end 225.38 126.5) (width 0.6) (layer "F.Cu") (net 8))
 (segment (start 223 123.5) (end 223 126.34) (width 0.6) (layer "F.Cu") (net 7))
 (segment (start 224.35 114.595) (end 222.9 114.595) (width 0.6) (layer "F.Cu") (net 7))
 (segment (start 223 126.34) (end 222.84 126.5) (width 0.6) (layer "F.Cu") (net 7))
 (segment (start 221 121.5) (end 223 123.5) (width 0.6) (layer "F.Cu") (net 7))
 (segment (start 221 116.495) (end 221 121.5) (width 0.6) (layer "F.Cu") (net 7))
 (segment (start 222.9 114.595) (end 221 116.495) (width 0.6) (layer "F.Cu") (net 7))
 (segment (start 229.61 117.725) (end 229.61 125.65) (width 0.6) (layer "F.Cu") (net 4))
 (segment (start 227.603 114.538) (end 227.603 112.925416) (width 0.6) (layer "F.Cu") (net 4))
 (segment (start 231.65 117.135) (end 230.2 117.135) (width 0.6) (layer "F.Cu") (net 4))
 (segment (start 214.001 107.201) (end 210.5 103.7) (width 0.6) (layer "F.Cu") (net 4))
 (segment (start 230.2 117.135) (end 227.603 114.538) (width 0.6) (layer "F.Cu") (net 4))
 (segment (start 220.701 107.201) (end 214.001 107.201) (width 0.6) (layer "F.Cu") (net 4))
 (segment (start 231.65 117.135) (end 230.2 117.135) (width 0.6) (layer "F.Cu") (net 4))
 (segment (start 210.5 103.7) (end 210.5 103) (width 0.6) (layer "F.Cu") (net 4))
 (segment (start 224.85 111.35) (end 220.701 107.201) (width 0.6) (layer "F.Cu") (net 4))
 (segment (start 227.603 112.925416) (end 226.027584 111.35) (width 0.6) (layer "F.Cu") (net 4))
 (segment (start 230.2 117.135) (end 229.61 117.725) (width 0.6) (layer "F.Cu") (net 4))
 (segment (start 226.027584 111.35) (end 224.85 111.35) (width 0.6) (layer "F.Cu") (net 4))
 (segment (start 229.61 125.65) (end 230.46 126.5) (width 0.6) (layer "F.Cu") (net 4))
 (segment (start 222.9 119.127208) (end 227.92 124.147208) (width 0.6) (layer "F.Cu") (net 9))
 (segment (start 224.35 117.135) (end 223.243 117.135) (width 0.6) (layer "F.Cu") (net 9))
 (segment (start 227.92 124.147208) (end 227.92 126.5) (width 0.6) (layer "F.Cu") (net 9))
 (segment (start 223.243 117.135) (end 222.9 117.478) (width 0.6) (layer "F.Cu") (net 9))
 (segment (start 222.9 117.478) (end 222.9 119.127208) (width 0.6) (layer "F.Cu") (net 9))
 (segment (start 231.65 122.61) (end 235.54 126.5) (width 0.6) (layer "F.Cu") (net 3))
 (segment (start 231.65 118.405) (end 231.65 122.61) (width 0.6) (layer "F.Cu") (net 3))
 (segment (start 230.656 115.865) (end 231.65 115.865) (width 0.6) (layer "F.Cu") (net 5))
 (segment (start 234.451 127.951) (end 233 126.5) (width 0.6) (layer "F.Cu") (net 5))
 (segment (start 217.001 104.699) (end 219.49 104.699) (width 0.6) (layer "F.Cu") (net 5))
 (segment (start 215 106) (end 215.7 106) (width 0.6) (layer "F.Cu") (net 5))
 (segment (start 219.49 104.699) (end 225.241 110.45) (width 0.6) (layer "F.Cu") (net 5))
 (segment (start 239.531 127.101024) (end 238.681024 127.951) (width 0.6) (layer "F.Cu") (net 5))
 (segment (start 228.55 113.759) (end 230.656 115.865) (width 0.6) (layer "F.Cu") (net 5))
 (segment (start 232.757 115.865) (end 239.531 122.639) (width 0.6) (layer "F.Cu") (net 5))
 (segment (start 228.55 112.504416) (end 228.55 113.759) (width 0.6) (layer "F.Cu") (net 5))
 (segment (start 225.241 110.45) (end 226.495584 110.45) (width 0.6) (layer "F.Cu") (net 5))
 (segment (start 226.495584 110.45) (end 228.55 112.504416) (width 0.6) (layer "F.Cu") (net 5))
 (segment (start 215.7 106) (end 217.001 104.699) (width 0.6) (layer "F.Cu") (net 5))
 (segment (start 239.531 122.639) (end 239.531 127.101024) (width 0.6) (layer "F.Cu") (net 5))
 (segment (start 238.681024 127.951) (end 234.451 127.951) (width 0.6) (layer "F.Cu") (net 5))
 (segment (start 231.65 115.865) (end 232.757 115.865) (width 0.6) (layer "F.Cu") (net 5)))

